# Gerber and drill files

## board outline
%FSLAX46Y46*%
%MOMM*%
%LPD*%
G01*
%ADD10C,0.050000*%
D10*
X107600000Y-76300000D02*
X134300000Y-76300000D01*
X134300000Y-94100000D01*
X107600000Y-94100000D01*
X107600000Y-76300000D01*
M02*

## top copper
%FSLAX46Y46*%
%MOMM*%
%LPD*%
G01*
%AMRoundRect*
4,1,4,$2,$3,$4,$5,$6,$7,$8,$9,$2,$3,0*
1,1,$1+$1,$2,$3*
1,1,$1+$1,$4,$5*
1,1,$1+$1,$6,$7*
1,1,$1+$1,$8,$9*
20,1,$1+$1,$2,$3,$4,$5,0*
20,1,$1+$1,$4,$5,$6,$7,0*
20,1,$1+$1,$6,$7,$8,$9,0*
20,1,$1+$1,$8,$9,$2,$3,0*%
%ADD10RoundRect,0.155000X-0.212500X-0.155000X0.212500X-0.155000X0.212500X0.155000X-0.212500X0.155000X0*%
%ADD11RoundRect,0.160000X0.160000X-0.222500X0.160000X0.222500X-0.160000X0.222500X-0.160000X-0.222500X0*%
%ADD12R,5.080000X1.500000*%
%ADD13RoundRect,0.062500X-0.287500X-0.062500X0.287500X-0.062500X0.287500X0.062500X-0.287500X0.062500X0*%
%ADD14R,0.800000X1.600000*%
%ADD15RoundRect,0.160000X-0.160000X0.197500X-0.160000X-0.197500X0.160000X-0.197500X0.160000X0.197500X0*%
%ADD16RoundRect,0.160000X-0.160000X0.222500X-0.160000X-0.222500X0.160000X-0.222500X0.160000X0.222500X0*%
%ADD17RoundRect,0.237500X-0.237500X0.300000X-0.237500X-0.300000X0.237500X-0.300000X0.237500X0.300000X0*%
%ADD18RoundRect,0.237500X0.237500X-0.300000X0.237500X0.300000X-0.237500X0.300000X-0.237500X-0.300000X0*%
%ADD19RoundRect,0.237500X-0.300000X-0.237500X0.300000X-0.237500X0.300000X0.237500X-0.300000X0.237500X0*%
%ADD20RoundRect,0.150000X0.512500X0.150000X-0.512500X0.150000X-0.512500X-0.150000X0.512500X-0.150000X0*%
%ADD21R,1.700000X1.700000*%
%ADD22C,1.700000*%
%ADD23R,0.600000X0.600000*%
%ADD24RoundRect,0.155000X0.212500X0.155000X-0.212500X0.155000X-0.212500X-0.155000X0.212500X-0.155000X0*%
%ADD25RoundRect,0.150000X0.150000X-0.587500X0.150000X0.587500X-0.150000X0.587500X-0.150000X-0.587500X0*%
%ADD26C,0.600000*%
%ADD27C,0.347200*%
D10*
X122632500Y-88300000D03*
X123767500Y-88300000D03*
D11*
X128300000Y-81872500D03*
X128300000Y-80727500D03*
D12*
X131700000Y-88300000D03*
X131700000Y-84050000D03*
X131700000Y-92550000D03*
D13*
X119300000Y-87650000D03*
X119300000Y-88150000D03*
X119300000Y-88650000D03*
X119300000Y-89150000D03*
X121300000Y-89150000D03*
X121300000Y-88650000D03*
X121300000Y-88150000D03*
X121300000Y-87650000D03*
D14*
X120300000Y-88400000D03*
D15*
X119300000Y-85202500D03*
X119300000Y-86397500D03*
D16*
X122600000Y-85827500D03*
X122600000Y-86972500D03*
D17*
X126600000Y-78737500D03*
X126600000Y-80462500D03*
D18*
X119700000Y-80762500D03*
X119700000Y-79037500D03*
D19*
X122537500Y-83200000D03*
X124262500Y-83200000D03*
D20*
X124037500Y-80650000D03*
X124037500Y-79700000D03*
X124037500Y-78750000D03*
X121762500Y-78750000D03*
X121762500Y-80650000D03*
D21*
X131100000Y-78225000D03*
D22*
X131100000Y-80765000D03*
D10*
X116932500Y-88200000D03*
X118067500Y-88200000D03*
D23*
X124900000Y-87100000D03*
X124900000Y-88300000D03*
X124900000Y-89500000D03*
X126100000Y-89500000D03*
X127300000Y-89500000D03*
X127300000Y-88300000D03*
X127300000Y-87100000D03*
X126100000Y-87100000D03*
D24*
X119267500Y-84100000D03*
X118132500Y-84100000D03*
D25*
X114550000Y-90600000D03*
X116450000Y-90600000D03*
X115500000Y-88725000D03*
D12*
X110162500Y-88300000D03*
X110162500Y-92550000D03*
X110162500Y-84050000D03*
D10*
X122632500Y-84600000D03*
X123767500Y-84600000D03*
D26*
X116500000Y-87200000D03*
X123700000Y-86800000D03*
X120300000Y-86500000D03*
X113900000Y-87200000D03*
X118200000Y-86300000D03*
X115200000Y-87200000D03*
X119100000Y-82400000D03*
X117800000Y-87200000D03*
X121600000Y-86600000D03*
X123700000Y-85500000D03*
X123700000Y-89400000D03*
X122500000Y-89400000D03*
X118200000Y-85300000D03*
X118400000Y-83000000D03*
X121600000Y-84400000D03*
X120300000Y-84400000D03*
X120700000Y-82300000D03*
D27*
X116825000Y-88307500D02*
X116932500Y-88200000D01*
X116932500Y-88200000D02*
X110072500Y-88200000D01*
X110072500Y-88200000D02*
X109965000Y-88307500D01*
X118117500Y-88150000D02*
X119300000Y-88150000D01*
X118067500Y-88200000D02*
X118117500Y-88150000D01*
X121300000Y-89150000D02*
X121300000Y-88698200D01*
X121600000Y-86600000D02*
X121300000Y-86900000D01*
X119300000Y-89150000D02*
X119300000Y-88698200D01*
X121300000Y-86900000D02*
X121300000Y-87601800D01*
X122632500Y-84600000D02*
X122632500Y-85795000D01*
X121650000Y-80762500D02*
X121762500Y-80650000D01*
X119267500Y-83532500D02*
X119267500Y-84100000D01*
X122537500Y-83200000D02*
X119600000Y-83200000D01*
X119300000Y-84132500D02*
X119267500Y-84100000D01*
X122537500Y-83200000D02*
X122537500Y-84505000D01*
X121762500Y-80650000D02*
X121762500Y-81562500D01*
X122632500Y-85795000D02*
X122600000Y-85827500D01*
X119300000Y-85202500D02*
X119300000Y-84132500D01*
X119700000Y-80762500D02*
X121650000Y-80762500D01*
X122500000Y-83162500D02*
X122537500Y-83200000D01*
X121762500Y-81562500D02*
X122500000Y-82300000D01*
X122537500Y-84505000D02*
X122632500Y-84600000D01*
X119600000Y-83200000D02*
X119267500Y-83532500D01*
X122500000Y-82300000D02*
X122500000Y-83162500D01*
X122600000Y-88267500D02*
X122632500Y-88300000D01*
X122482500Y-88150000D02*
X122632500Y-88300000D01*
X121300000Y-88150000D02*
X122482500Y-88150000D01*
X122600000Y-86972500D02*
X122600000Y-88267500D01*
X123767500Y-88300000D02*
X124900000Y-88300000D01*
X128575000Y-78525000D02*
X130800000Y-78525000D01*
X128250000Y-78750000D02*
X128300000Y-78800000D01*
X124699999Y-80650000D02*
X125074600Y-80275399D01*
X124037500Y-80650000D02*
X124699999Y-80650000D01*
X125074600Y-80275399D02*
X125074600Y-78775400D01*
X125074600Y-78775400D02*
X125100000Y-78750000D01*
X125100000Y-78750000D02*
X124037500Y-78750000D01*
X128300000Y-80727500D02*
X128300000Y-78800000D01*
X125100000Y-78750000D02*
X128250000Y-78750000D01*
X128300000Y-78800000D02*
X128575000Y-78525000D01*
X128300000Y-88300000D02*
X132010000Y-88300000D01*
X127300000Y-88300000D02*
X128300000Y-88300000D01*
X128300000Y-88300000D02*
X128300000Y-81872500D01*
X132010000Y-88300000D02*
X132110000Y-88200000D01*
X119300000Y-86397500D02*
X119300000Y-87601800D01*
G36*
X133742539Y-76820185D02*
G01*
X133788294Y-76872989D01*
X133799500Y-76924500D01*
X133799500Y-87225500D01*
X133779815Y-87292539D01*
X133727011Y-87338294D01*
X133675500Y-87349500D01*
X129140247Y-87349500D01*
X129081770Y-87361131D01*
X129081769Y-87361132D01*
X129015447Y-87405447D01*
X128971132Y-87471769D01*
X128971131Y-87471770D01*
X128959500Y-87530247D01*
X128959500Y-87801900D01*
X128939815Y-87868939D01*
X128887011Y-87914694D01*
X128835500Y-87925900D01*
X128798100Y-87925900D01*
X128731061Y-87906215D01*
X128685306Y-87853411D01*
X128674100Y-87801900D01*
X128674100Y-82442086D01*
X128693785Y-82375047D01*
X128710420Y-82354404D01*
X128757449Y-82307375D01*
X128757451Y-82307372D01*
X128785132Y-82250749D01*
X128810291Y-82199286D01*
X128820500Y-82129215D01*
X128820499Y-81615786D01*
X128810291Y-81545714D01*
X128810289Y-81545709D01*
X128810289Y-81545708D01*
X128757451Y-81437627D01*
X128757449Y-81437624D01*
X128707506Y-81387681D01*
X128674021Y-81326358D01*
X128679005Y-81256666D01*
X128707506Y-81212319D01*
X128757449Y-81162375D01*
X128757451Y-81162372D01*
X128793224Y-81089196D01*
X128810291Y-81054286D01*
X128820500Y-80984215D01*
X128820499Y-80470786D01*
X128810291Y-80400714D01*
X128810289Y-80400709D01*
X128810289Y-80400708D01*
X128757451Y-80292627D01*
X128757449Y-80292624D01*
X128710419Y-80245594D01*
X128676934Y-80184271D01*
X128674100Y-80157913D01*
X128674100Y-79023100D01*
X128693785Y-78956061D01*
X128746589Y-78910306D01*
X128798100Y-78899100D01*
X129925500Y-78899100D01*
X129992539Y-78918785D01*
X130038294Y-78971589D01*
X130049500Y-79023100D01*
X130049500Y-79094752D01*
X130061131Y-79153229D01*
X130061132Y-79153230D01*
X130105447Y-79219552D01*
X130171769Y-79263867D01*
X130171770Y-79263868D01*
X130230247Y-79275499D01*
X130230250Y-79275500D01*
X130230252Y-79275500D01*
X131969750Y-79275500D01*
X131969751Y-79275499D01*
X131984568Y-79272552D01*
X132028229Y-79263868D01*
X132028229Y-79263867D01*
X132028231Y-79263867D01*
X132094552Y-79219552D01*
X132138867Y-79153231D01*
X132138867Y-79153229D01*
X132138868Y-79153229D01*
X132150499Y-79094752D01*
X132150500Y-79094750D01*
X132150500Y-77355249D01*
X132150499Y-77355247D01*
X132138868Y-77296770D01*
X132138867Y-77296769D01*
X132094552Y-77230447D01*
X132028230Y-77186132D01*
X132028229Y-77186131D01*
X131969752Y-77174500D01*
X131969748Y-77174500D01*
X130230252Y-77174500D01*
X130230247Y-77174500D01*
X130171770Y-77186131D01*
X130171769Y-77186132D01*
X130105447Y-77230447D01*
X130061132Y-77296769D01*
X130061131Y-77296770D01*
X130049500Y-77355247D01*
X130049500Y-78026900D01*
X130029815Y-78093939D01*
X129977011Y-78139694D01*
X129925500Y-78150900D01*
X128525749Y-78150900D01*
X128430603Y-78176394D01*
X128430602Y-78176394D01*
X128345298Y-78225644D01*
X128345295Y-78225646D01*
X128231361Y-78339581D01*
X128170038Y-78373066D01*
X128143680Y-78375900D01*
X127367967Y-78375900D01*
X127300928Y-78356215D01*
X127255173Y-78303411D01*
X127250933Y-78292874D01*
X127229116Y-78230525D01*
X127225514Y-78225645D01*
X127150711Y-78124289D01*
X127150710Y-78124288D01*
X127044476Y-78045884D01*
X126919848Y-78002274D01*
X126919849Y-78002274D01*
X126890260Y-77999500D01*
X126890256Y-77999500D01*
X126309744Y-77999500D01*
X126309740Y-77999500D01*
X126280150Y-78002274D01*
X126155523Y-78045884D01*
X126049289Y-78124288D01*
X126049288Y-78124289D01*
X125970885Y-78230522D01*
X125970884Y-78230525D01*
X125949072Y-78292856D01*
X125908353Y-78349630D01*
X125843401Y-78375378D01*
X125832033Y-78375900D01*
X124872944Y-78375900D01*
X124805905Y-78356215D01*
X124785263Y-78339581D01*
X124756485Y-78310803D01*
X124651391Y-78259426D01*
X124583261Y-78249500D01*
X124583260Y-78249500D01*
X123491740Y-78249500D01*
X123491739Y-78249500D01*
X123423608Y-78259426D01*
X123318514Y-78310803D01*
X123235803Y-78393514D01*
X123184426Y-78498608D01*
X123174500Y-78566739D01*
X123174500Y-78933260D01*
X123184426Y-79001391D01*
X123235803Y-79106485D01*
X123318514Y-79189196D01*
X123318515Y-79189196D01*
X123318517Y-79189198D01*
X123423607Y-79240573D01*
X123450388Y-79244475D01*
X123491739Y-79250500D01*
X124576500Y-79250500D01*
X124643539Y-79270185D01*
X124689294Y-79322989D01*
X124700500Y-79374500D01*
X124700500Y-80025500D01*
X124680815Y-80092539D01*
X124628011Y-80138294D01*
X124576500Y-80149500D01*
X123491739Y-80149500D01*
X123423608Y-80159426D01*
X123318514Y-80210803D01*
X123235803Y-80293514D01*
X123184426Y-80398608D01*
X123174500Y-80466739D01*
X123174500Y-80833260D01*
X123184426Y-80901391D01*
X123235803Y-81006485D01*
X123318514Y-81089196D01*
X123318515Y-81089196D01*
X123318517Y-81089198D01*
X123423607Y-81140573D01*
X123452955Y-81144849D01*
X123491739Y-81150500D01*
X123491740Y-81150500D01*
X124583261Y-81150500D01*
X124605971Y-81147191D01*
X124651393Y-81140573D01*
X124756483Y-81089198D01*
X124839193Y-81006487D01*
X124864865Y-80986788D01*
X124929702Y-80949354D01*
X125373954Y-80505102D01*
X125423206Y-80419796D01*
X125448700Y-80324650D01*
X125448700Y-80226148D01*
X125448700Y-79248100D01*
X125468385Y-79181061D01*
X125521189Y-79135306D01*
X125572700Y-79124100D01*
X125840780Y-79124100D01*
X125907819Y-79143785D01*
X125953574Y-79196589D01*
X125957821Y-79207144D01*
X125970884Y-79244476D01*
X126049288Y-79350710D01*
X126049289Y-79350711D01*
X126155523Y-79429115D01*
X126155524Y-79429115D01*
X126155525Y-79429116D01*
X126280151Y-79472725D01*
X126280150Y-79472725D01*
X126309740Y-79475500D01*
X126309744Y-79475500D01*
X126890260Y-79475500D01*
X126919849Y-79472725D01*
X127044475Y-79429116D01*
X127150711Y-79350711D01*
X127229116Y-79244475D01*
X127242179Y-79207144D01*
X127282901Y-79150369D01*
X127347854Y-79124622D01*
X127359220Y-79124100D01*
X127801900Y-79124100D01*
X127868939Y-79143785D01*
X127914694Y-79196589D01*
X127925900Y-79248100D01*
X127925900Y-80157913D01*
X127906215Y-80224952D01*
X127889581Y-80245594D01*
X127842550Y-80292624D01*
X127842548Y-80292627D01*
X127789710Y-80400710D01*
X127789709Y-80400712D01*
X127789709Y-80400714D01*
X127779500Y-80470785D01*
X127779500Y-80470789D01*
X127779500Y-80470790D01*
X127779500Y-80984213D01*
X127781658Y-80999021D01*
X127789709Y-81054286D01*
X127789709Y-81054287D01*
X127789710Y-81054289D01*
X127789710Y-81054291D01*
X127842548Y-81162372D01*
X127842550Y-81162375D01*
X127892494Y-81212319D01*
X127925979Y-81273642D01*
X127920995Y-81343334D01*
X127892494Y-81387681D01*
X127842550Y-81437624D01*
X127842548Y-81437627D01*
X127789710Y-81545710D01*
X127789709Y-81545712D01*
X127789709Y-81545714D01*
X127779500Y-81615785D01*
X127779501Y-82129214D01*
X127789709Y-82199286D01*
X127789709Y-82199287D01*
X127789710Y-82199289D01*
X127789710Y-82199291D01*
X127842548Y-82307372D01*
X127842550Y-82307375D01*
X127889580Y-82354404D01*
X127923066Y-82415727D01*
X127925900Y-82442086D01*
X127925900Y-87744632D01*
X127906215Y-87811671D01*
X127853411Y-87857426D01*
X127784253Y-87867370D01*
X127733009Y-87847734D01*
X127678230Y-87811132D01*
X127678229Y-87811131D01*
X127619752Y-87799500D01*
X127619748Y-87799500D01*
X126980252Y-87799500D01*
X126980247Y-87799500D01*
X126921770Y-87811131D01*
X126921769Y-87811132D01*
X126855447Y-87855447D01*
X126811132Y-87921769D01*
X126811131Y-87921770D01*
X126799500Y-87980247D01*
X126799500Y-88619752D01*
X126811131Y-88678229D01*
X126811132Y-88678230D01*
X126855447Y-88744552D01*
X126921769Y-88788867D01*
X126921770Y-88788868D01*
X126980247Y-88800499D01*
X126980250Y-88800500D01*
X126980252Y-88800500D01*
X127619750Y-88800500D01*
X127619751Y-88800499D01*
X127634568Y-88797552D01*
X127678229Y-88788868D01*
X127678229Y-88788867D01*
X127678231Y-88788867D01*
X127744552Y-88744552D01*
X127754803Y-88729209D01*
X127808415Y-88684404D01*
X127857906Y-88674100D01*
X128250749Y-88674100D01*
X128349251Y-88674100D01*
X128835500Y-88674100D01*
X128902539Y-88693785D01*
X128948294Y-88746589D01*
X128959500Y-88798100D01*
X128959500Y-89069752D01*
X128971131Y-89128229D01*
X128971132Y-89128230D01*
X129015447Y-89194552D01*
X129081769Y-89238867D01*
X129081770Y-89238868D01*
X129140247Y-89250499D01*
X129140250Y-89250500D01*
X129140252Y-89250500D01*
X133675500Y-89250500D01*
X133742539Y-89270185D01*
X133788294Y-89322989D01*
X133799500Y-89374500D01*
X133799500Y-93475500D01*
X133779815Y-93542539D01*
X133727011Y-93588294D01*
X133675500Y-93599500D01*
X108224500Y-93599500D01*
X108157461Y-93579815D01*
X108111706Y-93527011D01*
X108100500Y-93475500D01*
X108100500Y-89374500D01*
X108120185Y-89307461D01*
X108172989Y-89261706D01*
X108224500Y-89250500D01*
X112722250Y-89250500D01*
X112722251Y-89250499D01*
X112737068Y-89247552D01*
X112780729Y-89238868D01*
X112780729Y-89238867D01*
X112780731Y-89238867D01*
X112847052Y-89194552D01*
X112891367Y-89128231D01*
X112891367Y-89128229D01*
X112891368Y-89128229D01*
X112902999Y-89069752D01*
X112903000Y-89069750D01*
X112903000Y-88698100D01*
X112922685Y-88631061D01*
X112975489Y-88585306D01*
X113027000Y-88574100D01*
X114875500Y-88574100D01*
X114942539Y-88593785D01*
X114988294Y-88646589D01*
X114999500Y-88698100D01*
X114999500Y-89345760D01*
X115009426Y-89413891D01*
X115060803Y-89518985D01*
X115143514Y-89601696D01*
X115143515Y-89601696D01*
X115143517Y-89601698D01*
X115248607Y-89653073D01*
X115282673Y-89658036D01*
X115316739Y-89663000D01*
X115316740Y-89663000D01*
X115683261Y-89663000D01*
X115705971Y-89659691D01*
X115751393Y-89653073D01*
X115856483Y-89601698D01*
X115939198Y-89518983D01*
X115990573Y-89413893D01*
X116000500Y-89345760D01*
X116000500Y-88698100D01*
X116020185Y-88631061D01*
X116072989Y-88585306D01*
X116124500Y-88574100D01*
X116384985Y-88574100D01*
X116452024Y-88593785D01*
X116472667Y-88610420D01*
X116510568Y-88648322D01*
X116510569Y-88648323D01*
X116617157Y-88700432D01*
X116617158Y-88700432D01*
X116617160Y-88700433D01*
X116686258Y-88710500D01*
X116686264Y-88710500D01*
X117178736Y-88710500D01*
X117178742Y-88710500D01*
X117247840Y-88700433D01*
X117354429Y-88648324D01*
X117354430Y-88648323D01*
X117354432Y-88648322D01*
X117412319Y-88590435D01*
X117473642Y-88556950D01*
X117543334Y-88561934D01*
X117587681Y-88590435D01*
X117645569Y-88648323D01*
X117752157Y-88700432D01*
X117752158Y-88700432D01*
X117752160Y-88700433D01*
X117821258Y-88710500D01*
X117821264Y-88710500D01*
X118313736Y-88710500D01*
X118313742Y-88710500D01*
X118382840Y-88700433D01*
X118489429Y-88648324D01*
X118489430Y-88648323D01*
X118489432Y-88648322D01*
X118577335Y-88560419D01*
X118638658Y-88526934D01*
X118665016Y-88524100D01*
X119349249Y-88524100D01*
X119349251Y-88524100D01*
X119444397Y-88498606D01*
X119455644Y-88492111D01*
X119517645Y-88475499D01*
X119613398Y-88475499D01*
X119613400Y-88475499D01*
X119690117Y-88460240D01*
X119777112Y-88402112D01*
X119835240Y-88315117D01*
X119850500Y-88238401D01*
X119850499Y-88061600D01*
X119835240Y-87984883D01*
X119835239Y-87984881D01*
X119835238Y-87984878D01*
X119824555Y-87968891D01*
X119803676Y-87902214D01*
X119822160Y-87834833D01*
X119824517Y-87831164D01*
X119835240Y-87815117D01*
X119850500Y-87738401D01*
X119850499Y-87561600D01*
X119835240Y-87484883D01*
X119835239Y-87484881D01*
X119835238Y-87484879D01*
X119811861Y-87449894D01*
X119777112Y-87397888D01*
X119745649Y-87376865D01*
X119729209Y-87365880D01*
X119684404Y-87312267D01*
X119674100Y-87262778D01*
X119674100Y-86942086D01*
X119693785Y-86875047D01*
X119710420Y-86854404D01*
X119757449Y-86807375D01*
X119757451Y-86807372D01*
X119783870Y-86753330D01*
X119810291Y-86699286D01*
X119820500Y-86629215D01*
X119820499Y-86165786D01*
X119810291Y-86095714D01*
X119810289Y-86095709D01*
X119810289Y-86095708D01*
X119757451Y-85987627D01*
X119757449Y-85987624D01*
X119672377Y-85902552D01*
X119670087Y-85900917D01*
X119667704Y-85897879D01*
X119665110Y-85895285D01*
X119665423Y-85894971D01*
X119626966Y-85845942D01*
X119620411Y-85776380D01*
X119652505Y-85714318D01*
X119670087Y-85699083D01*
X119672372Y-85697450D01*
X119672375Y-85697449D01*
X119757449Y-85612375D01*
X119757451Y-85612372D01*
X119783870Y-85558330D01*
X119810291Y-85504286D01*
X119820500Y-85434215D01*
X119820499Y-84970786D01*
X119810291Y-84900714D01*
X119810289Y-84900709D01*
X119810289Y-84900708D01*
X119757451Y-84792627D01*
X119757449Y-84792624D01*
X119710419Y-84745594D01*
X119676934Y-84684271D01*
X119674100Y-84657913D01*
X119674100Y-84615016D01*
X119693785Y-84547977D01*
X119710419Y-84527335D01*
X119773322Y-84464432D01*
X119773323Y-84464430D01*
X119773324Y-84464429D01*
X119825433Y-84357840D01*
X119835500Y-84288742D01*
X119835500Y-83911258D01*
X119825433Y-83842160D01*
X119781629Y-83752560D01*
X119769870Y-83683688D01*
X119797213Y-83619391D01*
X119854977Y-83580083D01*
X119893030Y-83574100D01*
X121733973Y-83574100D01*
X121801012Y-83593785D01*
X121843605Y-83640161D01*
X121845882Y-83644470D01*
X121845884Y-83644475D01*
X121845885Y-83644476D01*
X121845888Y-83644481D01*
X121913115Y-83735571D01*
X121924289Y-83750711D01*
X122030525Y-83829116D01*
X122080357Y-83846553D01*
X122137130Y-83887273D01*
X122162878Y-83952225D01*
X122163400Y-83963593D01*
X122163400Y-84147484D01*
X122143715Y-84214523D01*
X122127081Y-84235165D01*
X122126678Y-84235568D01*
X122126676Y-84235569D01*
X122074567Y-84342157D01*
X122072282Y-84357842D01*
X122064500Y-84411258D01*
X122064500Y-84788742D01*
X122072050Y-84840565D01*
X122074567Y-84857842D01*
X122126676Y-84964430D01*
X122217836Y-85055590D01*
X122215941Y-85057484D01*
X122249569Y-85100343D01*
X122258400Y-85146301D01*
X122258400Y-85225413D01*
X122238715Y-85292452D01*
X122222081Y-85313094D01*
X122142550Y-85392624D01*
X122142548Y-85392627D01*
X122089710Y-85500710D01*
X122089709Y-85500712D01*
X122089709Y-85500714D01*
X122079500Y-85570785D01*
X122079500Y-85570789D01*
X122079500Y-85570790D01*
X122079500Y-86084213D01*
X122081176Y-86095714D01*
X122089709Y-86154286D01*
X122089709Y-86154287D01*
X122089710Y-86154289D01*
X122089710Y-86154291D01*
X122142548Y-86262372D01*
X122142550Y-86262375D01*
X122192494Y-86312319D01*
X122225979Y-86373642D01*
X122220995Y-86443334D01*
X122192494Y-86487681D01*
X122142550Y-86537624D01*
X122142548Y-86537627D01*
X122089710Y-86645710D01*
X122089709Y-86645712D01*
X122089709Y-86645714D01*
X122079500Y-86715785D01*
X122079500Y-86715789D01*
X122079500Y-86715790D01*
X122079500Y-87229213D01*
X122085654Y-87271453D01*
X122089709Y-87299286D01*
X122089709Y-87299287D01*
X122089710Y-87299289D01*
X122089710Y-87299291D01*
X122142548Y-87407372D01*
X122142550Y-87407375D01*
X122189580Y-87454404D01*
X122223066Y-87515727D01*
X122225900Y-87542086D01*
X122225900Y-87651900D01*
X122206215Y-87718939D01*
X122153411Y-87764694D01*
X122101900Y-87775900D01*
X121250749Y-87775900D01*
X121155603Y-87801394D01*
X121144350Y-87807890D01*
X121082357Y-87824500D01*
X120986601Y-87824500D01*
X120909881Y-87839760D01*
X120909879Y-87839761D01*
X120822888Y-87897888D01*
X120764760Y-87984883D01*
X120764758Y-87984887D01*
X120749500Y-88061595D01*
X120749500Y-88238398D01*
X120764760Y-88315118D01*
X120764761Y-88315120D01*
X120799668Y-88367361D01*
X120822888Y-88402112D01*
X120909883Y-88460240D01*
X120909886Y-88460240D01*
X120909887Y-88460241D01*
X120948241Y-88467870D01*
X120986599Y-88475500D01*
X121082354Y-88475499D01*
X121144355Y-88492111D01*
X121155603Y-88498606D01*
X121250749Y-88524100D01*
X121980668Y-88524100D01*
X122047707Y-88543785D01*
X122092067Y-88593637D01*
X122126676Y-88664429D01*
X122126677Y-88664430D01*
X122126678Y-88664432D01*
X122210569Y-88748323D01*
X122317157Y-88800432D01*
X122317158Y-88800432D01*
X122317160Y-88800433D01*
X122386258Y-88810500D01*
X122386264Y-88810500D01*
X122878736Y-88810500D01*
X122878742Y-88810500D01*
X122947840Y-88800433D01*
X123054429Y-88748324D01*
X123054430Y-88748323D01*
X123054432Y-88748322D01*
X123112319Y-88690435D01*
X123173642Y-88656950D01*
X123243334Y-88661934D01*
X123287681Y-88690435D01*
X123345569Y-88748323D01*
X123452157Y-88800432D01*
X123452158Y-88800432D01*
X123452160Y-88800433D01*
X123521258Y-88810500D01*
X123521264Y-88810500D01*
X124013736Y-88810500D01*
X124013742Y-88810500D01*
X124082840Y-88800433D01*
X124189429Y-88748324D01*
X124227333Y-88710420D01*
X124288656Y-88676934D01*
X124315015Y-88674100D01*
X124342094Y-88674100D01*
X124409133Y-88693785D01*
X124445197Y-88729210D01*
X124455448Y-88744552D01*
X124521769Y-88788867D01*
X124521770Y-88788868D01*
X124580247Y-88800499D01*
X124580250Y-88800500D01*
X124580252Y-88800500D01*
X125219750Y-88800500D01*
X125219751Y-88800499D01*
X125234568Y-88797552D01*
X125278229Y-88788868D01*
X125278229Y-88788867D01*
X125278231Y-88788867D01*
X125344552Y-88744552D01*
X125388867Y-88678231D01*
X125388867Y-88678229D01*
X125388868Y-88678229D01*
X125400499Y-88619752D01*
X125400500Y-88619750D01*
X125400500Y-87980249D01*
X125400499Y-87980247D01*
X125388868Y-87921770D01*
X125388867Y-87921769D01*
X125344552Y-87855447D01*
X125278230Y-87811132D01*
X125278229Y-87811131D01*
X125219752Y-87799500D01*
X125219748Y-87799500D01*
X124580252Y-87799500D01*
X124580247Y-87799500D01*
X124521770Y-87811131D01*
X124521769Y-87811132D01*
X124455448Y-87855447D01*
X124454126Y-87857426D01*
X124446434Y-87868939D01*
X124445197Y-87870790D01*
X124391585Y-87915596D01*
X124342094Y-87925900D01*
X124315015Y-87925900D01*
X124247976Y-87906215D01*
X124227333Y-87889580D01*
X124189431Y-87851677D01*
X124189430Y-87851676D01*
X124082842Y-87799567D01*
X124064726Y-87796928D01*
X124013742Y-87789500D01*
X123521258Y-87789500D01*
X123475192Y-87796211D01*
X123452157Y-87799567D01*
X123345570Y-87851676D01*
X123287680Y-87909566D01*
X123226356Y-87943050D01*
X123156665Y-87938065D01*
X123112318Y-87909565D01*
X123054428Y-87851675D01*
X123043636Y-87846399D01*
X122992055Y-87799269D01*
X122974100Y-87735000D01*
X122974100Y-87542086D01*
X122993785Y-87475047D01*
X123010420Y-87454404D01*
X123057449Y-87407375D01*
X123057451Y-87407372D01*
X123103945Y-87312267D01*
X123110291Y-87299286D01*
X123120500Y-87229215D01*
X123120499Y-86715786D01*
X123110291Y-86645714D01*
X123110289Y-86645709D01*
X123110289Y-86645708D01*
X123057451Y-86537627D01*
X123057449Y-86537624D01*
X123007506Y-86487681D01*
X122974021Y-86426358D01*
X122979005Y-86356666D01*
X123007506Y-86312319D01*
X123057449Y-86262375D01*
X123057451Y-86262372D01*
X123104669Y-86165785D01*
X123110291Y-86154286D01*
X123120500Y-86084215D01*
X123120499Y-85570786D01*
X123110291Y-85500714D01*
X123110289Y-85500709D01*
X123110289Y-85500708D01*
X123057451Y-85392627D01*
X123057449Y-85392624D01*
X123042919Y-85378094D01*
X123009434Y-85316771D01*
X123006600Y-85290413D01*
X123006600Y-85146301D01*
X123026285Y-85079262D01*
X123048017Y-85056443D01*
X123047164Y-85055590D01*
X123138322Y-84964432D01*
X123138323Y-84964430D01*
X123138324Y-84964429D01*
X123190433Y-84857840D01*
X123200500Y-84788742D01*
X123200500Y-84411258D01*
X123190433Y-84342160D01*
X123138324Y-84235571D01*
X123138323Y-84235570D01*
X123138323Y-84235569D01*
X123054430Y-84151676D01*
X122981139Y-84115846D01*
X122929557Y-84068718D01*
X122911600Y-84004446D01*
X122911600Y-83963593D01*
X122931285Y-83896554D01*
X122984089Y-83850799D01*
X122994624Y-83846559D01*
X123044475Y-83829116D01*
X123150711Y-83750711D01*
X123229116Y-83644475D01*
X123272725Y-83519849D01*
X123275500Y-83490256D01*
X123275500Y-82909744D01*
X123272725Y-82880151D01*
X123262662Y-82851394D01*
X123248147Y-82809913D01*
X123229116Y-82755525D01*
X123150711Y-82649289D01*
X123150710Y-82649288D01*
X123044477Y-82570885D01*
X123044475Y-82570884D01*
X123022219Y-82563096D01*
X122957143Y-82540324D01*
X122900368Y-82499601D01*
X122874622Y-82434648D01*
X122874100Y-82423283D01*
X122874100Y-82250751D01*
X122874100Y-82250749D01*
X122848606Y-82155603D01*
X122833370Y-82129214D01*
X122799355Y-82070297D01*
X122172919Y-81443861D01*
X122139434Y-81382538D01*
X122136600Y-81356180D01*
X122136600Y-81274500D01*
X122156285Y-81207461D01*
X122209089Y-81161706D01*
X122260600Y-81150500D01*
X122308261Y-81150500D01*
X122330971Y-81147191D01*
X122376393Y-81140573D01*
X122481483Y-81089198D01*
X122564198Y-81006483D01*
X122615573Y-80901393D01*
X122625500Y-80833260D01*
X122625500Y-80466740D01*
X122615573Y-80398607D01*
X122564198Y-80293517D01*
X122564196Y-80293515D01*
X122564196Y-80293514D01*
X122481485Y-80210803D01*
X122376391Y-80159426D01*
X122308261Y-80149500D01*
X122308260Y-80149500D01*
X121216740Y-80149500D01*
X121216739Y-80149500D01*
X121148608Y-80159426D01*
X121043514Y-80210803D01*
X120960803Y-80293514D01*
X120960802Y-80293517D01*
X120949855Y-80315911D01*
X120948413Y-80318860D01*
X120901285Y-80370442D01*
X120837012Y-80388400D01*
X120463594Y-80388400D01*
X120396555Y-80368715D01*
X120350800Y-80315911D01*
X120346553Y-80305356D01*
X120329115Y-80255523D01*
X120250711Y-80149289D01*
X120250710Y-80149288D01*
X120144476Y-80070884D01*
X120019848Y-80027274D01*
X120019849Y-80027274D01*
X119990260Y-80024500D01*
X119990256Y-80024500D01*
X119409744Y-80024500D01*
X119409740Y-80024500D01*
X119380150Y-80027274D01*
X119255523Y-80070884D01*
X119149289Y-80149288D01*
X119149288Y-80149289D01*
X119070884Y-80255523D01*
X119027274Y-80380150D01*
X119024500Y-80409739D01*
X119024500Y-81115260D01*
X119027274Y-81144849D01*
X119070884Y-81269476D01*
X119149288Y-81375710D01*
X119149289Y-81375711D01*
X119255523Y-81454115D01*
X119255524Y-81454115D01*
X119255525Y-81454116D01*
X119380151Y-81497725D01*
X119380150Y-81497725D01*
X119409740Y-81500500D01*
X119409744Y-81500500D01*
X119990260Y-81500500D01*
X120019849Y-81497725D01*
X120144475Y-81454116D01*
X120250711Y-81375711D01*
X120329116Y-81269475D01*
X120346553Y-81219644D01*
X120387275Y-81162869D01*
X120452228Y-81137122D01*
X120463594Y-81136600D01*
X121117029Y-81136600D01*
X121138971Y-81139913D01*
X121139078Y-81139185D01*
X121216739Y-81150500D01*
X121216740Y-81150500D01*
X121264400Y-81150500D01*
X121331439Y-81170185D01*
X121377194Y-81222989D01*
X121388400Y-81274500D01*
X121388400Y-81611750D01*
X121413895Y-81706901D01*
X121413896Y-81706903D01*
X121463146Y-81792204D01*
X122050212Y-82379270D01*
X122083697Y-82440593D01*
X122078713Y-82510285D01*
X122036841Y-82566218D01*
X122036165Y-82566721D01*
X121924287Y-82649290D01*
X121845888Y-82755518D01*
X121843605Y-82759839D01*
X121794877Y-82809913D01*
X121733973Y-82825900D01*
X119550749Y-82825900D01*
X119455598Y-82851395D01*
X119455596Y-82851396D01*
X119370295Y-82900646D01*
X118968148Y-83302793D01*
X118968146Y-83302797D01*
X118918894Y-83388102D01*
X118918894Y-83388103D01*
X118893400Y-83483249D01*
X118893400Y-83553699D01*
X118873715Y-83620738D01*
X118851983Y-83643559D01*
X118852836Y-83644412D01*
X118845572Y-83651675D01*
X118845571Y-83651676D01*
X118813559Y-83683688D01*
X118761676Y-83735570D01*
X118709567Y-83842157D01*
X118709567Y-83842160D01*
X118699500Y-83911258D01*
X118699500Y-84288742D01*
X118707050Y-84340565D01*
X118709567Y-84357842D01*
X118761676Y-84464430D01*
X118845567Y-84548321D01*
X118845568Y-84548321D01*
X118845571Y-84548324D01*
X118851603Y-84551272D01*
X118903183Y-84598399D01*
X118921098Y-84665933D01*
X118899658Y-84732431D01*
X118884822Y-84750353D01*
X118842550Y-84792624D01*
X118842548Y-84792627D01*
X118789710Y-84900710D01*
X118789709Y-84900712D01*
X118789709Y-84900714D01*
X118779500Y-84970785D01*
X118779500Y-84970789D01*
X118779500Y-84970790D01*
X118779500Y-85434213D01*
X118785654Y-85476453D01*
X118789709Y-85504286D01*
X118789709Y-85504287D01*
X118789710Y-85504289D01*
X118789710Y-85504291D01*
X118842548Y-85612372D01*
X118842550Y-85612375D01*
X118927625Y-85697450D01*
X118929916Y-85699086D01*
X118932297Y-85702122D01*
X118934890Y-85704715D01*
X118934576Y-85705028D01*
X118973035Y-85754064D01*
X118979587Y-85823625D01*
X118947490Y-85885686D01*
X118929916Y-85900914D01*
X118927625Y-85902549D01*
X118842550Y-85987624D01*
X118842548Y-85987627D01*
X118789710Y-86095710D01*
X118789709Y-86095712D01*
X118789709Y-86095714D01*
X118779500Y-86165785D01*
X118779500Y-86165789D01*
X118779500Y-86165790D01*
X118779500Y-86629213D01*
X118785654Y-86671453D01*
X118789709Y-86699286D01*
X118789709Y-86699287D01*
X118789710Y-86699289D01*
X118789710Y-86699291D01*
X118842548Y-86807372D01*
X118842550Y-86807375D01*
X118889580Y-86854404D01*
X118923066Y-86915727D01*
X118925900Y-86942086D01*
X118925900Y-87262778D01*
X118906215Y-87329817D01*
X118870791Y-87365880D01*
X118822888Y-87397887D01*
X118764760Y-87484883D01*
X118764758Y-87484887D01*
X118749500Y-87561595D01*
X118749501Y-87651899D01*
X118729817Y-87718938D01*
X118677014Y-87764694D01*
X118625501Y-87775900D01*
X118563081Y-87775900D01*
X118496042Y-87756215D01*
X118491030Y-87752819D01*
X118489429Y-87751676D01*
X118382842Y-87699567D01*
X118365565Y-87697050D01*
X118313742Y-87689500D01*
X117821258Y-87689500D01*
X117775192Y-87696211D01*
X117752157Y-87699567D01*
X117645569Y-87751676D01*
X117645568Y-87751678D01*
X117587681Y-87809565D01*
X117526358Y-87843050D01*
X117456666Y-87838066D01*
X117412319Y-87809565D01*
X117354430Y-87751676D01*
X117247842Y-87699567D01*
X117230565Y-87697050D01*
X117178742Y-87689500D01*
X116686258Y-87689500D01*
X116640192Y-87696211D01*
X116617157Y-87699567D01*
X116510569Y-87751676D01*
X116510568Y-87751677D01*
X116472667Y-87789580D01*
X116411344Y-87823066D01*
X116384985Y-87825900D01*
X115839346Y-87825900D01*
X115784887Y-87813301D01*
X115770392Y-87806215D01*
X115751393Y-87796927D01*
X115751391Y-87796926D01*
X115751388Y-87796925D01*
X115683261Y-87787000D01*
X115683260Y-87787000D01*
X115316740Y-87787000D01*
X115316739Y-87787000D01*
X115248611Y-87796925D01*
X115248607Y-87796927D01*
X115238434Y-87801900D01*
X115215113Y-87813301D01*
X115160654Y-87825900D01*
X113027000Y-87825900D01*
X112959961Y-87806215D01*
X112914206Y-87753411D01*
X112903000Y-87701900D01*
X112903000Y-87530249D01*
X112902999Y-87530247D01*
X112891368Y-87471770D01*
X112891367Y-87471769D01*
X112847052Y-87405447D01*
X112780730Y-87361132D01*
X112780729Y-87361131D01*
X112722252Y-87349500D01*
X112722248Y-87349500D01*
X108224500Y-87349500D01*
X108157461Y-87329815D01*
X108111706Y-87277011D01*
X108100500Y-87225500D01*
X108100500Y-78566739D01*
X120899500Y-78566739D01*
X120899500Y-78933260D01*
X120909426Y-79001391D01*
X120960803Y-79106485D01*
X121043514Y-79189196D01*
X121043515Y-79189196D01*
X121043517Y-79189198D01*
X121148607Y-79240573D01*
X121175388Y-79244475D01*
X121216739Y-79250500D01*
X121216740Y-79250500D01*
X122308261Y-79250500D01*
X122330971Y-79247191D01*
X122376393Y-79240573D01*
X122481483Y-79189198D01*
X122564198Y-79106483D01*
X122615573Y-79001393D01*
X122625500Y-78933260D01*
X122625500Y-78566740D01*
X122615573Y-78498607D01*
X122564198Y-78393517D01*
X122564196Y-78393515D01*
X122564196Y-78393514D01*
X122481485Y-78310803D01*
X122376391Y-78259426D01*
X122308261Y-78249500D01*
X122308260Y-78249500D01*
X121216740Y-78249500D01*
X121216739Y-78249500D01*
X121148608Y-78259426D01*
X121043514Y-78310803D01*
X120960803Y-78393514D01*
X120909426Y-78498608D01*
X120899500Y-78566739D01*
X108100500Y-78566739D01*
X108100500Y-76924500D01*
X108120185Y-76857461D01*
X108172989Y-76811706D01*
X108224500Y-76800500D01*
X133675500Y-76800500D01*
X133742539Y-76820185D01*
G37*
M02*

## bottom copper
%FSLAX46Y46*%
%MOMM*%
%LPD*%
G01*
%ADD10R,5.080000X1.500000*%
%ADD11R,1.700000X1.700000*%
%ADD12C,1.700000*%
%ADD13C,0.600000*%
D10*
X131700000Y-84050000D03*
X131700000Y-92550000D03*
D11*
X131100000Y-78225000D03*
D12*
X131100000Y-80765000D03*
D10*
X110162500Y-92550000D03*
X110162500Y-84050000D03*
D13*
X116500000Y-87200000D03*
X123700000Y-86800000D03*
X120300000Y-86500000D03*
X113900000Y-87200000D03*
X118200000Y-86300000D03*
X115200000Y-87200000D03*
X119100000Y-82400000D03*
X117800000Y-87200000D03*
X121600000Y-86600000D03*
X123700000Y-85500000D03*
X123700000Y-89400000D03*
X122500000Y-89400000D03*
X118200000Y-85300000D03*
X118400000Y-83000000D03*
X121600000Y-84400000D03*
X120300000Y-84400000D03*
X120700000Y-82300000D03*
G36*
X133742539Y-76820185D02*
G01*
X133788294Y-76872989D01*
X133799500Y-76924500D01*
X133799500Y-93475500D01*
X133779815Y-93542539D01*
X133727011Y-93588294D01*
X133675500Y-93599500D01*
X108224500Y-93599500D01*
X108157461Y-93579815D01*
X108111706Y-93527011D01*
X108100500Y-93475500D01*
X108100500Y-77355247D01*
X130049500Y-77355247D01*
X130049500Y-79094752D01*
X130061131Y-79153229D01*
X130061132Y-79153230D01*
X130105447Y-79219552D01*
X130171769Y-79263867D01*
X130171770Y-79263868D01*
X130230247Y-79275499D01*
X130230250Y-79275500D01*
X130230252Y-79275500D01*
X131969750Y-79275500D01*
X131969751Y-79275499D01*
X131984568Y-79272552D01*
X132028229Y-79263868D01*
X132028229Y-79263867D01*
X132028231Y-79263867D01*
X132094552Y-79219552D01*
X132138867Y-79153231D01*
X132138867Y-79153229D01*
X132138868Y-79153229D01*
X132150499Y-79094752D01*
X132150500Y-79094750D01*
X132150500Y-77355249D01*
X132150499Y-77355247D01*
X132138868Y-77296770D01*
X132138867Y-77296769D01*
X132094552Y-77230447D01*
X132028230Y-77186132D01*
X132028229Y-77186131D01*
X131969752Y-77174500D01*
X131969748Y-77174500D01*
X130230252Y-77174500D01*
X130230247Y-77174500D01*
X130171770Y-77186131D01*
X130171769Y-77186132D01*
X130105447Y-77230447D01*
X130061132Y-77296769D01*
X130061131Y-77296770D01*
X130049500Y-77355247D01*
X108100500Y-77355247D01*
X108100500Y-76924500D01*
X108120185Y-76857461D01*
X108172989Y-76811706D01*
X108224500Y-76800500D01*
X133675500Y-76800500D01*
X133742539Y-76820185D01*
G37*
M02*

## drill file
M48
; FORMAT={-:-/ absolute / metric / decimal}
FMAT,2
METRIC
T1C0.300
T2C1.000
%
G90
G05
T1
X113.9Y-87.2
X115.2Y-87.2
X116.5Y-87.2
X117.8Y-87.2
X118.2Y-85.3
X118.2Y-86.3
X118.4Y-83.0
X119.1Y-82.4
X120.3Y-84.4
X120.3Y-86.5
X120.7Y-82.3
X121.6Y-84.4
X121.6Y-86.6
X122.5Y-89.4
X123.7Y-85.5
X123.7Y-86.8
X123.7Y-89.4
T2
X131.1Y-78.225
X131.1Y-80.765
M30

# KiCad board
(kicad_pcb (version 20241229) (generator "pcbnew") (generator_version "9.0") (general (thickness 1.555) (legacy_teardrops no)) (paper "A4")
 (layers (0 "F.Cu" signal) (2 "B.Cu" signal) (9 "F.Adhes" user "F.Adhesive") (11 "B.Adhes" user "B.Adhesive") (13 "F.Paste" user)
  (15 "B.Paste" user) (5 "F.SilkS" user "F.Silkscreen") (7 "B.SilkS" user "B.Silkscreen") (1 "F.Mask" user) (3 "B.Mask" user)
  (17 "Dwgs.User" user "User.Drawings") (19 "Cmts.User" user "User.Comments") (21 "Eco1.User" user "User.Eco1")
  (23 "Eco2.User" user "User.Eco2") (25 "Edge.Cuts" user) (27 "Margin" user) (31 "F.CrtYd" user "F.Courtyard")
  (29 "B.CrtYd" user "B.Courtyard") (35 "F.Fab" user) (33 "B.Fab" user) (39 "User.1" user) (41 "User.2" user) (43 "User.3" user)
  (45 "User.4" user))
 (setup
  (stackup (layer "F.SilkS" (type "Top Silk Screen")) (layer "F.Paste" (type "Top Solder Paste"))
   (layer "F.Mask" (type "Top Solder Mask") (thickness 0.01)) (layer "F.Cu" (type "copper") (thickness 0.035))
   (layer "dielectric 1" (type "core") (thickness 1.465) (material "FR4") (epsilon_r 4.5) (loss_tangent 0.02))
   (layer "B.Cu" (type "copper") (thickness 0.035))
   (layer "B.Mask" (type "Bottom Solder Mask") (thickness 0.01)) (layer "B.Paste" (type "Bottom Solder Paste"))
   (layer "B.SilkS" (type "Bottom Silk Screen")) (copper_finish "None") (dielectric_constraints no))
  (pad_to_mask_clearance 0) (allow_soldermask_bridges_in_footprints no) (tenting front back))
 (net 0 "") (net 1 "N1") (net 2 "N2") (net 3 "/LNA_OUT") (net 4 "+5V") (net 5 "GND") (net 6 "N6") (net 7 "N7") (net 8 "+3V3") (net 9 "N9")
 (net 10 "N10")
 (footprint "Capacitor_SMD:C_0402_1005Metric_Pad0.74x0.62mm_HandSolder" (layer "F.Cu") (at 123.2 88.3)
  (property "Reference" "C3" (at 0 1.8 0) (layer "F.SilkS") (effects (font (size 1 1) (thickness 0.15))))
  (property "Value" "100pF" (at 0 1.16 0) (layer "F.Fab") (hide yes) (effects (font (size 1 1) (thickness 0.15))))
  (pad "1" smd roundrect (at -0.5675 0) (size 0.735 0.62) (layers "F.Cu" "F.Mask" "F.Paste") (roundrect_rratio 0.25) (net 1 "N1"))
  (pad "2" smd roundrect (at 0.5675 0) (size 0.735 0.62) (layers "F.Cu" "F.Mask" "F.Paste") (roundrect_rratio 0.25) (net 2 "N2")))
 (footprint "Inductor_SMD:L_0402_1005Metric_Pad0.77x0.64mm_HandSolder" (layer "F.Cu") (at 128.3 81.3 90)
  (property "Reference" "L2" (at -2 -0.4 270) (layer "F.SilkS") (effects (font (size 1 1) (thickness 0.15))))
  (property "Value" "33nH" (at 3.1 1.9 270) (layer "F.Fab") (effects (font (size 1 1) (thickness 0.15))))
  (pad "1" smd roundrect (at -0.5725 0 90) (size 0.765 0.64) (layers "F.Cu" "F.Mask" "F.Paste") (roundrect_rratio 0.25) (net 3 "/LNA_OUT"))
  (pad "2" smd roundrect (at 0.5725 0 90) (size 0.765 0.64) (layers "F.Cu" "F.Mask" "F.Paste") (roundrect_rratio 0.25) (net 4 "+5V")))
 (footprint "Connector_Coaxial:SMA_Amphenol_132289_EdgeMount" (layer "F.Cu") (at 131.7 88.3)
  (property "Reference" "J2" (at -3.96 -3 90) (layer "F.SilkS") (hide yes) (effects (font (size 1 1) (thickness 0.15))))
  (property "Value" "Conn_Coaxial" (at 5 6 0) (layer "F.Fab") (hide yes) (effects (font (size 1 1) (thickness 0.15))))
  (pad "1" smd rect (at 0 0 90) (size 1.5 5.08) (layers "F.Cu" "F.Mask" "F.Paste") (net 3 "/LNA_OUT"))
  (pad "2" smd rect (at 0 -4.25 90) (size 1.5 5.08) (layers "F.Cu" "F.Mask" "F.Paste") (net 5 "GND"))
  (pad "2" smd rect (at 0 -4.25 90) (size 1.5 5.08) (layers "B.Cu" "B.Mask" "B.Paste") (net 5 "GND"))
  (pad "2" smd rect (at 0 4.25 90) (size 1.5 5.08) (layers "F.Cu" "F.Mask" "F.Paste") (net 5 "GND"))
  (pad "2" smd rect (at 0 4.25 90) (size 1.5 5.08) (layers "B.Cu" "B.Mask" "B.Paste") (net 5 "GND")))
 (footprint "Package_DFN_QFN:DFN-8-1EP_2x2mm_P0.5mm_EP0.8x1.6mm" (layer "F.Cu") (at 120.3 88.4)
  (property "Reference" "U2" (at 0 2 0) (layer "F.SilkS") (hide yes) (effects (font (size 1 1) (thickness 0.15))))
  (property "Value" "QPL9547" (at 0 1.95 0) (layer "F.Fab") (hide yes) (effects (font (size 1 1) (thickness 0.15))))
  (pad "" smd roundrect (at 0 0) (size 0.64 1.29) (layers "F.Paste") (roundrect_rratio 0.25))
  (pad "1" smd roundrect (at -1 -0.75) (size 0.7 0.25) (layers "F.Cu" "F.Mask" "F.Paste") (roundrect_rratio 0.25) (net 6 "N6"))
  (pad "2" smd roundrect (at -1 -0.25) (size 0.7 0.25) (layers "F.Cu" "F.Mask" "F.Paste") (roundrect_rratio 0.25) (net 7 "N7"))
  (pad "3" smd roundrect (at -1 0.25) (size 0.7 0.25) (layers "F.Cu" "F.Mask" "F.Paste") (roundrect_rratio 0.25) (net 5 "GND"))
  (pad "4" smd roundrect (at -1 0.75) (size 0.7 0.25) (layers "F.Cu" "F.Mask" "F.Paste") (roundrect_rratio 0.25) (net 5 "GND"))
  (pad "5" smd roundrect (at 1 0.75) (size 0.7 0.25) (layers "F.Cu" "F.Mask" "F.Paste") (roundrect_rratio 0.25) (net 5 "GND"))
  (pad "6" smd roundrect (at 1 0.25) (size 0.7 0.25) (layers "F.Cu" "F.Mask" "F.Paste") (roundrect_rratio 0.25) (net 5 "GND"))
  (pad "7" smd roundrect (at 1 -0.25) (size 0.7 0.25) (layers "F.Cu" "F.Mask" "F.Paste") (roundrect_rratio 0.25) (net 1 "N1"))
  (pad "8" smd roundrect (at 1 -0.75) (size 0.7 0.25) (layers "F.Cu" "F.Mask" "F.Paste") (roundrect_rratio 0.25) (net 5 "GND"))
  (pad "9" smd rect (at 0 0) (size 0.8 1.6) (layers "F.Cu" "F.Mask") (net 5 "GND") (zone_connect 2)))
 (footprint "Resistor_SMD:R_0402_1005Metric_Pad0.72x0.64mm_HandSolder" (layer "F.Cu") (at 119.3 85.8 -90)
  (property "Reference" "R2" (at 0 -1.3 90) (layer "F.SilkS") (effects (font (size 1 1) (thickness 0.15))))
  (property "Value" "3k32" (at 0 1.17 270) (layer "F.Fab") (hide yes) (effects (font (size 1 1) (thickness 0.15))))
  (pad "1" smd roundrect (at -0.5975 0 270) (size 0.715 0.64) (layers "F.Cu" "F.Mask" "F.Paste") (roundrect_rratio 0.25) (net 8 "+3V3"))
  (pad "2" smd roundrect (at 0.5975 0 270) (size 0.715 0.64) (layers "F.Cu" "F.Mask" "F.Paste") (roundrect_rratio 0.25) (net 6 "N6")))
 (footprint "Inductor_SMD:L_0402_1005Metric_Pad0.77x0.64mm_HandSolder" (layer "F.Cu") (at 122.6 86.4 -90)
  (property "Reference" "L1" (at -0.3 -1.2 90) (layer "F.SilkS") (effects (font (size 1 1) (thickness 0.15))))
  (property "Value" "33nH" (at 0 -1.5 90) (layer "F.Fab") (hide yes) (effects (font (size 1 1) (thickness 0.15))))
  (pad "1" smd roundrect (at -0.5725 0 270) (size 0.765 0.64) (layers "F.Cu" "F.Mask" "F.Paste") (roundrect_rratio 0.25) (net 8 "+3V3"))
  (pad "2" smd roundrect (at 0.5725 0 270) (size 0.765 0.64) (layers "F.Cu" "F.Mask" "F.Paste") (roundrect_rratio 0.25) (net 1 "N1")))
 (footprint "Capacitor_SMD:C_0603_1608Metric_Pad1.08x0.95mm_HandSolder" (layer "F.Cu") (at 126.6 79.6 -90)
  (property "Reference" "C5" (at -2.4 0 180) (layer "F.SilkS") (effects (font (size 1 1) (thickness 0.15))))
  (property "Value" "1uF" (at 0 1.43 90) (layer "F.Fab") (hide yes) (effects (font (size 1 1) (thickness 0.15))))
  (pad "1" smd roundrect (at -0.8625 0 270) (size 1.075 0.95) (layers "F.Cu" "F.Mask" "F.Paste") (roundrect_rratio 0.25) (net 4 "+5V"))
  (pad "2" smd roundrect (at 0.8625 0 270) (size 1.075 0.95) (layers "F.Cu" "F.Mask" "F.Paste") (roundrect_rratio 0.25) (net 5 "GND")))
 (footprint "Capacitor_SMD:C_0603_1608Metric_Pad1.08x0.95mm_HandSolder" (layer "F.Cu") (at 119.7 79.9 90)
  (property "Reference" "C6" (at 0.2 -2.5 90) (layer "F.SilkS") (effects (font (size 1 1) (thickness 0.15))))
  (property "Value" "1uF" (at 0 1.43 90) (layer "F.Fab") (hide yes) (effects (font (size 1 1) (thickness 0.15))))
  (pad "1" smd roundrect (at -0.8625 0 90) (size 1.075 0.95) (layers "F.Cu" "F.Mask" "F.Paste") (roundrect_rratio 0.25) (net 8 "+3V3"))
  (pad "2" smd roundrect (at 0.8625 0 90) (size 1.075 0.95) (layers "F.Cu" "F.Mask" "F.Paste") (roundrect_rratio 0.25) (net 5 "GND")))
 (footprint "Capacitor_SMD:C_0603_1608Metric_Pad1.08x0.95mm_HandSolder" (layer "F.Cu") (at 123.4 83.2)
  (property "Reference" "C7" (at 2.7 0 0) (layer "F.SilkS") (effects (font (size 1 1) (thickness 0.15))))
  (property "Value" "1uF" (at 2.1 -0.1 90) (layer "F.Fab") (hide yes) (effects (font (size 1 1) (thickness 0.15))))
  (pad "1" smd roundrect (at -0.8625 0) (size 1.075 0.95) (layers "F.Cu" "F.Mask" "F.Paste") (roundrect_rratio 0.25) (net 8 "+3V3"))
  (pad "2" smd roundrect (at 0.8625 0) (size 1.075 0.95) (layers "F.Cu" "F.Mask" "F.Paste") (roundrect_rratio 0.25) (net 5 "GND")))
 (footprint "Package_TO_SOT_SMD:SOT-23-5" (layer "F.Cu") (at 122.9 79.7 180)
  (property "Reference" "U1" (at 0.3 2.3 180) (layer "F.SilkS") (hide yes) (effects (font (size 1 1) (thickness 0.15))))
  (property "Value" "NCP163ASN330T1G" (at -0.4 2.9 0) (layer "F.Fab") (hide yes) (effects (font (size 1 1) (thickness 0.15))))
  (pad "1" smd roundrect (at -1.1375 -0.95 180) (size 1.325 0.6) (layers "F.Cu" "F.Mask" "F.Paste") (roundrect_rratio 0.25) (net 4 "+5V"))
  (pad "2" smd roundrect (at -1.1375 0 180) (size 1.325 0.6) (layers "F.Cu" "F.Mask" "F.Paste") (roundrect_rratio 0.25) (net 5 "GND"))
  (pad "3" smd roundrect (at -1.1375 0.95 180) (size 1.325 0.6) (layers "F.Cu" "F.Mask" "F.Paste") (roundrect_rratio 0.25) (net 4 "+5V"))
  (pad "4" smd roundrect (at 1.1375 0.95 180) (size 1.325 0.6) (layers "F.Cu" "F.Mask" "F.Paste") (roundrect_rratio 0.25) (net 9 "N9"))
  (pad "5" smd roundrect (at 1.1375 -0.95 180) (size 1.325 0.6) (layers "F.Cu" "F.Mask" "F.Paste") (roundrect_rratio 0.25) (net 8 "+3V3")))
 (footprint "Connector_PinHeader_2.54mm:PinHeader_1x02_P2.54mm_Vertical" (layer "F.Cu") (at 131.1 78.225)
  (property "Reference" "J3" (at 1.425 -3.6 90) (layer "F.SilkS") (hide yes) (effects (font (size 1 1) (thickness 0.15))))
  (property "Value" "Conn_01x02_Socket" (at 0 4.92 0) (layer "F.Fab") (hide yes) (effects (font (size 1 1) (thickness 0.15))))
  (pad "1" thru_hole rect (at 0 0) (size 1.7 1.7) (drill 1) (layers "*.Cu" "*.Mask") (remove_unused_layers no) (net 4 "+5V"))
  (pad "2" thru_hole circle (at 0 2.54) (size 1.7 1.7) (drill 1) (layers "*.Cu" "*.Mask") (remove_unused_layers no) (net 5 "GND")))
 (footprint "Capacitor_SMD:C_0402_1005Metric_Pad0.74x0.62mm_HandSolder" (layer "F.Cu") (at 117.5 88.2)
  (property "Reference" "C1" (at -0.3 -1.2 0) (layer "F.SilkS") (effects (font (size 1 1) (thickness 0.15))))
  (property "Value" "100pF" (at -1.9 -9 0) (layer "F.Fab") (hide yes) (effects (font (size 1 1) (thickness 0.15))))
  (pad "1" smd roundrect (at -0.5675 0) (size 0.735 0.62) (layers "F.Cu" "F.Mask" "F.Paste") (roundrect_rratio 0.25) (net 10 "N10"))
  (pad "2" smd roundrect (at 0.5675 0) (size 0.735 0.62) (layers "F.Cu" "F.Mask" "F.Paste") (roundrect_rratio 0.25) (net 7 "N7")))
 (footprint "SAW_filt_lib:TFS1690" (layer "F.Cu") (at 126.6 88.3 -90)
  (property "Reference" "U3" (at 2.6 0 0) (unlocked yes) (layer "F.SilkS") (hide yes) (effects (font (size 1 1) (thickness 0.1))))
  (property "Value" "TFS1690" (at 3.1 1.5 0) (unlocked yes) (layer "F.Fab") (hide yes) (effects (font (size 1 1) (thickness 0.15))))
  (pad "1" smd rect (at -1.2 1.7 270) (size 0.6 0.6) (layers "F.Cu" "F.Mask" "F.Paste") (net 5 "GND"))
  (pad "2" smd rect (at 0 1.7 270) (size 0.6 0.6) (layers "F.Cu" "F.Mask" "F.Paste") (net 2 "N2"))
  (pad "3" smd rect (at 1.2 1.7 270) (size 0.6 0.6) (layers "F.Cu" "F.Mask" "F.Paste") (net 5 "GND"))
  (pad "4" smd rect (at 1.2 0.5 270) (size 0.6 0.6) (layers "F.Cu" "F.Mask" "F.Paste") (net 5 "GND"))
  (pad "5" smd rect (at 1.2 -0.7 270) (size 0.6 0.6) (layers "F.Cu" "F.Mask" "F.Paste") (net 5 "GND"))
  (pad "6" smd rect (at 0 -0.7 270) (size 0.6 0.6) (layers "F.Cu" "F.Mask" "F.Paste") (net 3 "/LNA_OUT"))
  (pad "7" smd rect (at -1.2 -0.7 270) (size 0.6 0.6) (layers "F.Cu" "F.Mask" "F.Paste") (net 5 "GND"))
  (pad "8" smd rect (at -1.2 0.5 270) (size 0.6 0.6) (layers "F.Cu" "F.Mask" "F.Paste") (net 5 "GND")))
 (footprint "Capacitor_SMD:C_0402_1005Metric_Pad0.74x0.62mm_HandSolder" (layer "F.Cu") (at 118.7 84.1 180)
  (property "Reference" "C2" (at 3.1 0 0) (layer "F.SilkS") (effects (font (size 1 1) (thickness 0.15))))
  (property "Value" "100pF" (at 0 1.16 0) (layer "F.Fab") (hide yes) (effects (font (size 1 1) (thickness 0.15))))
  (pad "1" smd roundrect (at -0.5675 0 180) (size 0.735 0.62) (layers "F.Cu" "F.Mask" "F.Paste") (roundrect_rratio 0.25) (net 8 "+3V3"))
  (pad "2" smd roundrect (at 0.5675 0 180) (size 0.735 0.62) (layers "F.Cu" "F.Mask" "F.Paste") (roundrect_rratio 0.25) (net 5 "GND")))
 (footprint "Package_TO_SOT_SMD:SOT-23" (layer "F.Cu") (at 115.5 89.6625 90)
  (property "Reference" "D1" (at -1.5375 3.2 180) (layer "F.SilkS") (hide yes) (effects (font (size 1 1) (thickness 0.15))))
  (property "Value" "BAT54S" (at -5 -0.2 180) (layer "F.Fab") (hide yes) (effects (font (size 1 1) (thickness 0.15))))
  (pad "1" smd roundrect (at -0.9375 -0.95 90) (size 1.475 0.6) (layers "F.Cu" "F.Mask" "F.Paste") (roundrect_rratio 0.25) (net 5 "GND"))
  (pad "2" smd roundrect (at -0.9375 0.95 90) (size 1.475 0.6) (layers "F.Cu" "F.Mask" "F.Paste") (roundrect_rratio 0.25) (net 5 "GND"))
  (pad "3" smd roundrect (at 0.9375 0 90) (size 1.475 0.6) (layers "F.Cu" "F.Mask" "F.Paste") (roundrect_rratio 0.25) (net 10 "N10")))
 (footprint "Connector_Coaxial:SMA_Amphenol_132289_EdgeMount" (layer "F.Cu") (at 110.1625 88.3 180)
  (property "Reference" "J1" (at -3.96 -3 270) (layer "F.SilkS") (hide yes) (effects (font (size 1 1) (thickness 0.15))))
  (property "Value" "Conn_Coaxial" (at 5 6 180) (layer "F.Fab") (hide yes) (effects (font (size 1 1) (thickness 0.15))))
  (pad "1" smd rect (at 0 0 270) (size 1.5 5.08) (layers "F.Cu" "F.Mask" "F.Paste") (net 10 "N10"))
  (pad "2" smd rect (at 0 -4.25 270) (size 1.5 5.08) (layers "F.Cu" "F.Mask" "F.Paste") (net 5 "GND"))
  (pad "2" smd rect (at 0 -4.25 270) (size 1.5 5.08) (layers "B.Cu" "B.Mask" "B.Paste") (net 5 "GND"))
  (pad "2" smd rect (at 0 4.25 270) (size 1.5 5.08) (layers "F.Cu" "F.Mask" "F.Paste") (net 5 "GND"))
  (pad "2" smd rect (at 0 4.25 270) (size 1.5 5.08) (layers "B.Cu" "B.Mask" "B.Paste") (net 5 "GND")))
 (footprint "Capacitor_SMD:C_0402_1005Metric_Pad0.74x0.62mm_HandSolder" (layer "F.Cu") (at 123.2 84.6)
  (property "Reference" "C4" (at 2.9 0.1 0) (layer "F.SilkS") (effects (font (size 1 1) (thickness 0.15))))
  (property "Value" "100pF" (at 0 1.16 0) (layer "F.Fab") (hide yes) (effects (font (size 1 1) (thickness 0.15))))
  (pad "1" smd roundrect (at -0.5675 0) (size 0.735 0.62) (layers "F.Cu" "F.Mask" "F.Paste") (roundrect_rratio 0.25) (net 8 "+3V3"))
  (pad "2" smd roundrect (at 0.5675 0) (size 0.735 0.62) (layers "F.Cu" "F.Mask" "F.Paste") (roundrect_rratio 0.25) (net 5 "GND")))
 (gr_rect (start 107.6 76.3) (end 134.3 94.1) (stroke (width 0.05) (type default)) (fill no) (layer "Edge.Cuts"))
 (segment (start 116.825 88.3075) (end 116.9325 88.2) (width 0.3472) (layer "F.Cu") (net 10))
 (segment (start 116.9325 88.2) (end 110.0725 88.2) (width 0.3472) (layer "F.Cu") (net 10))
 (segment (start 110.0725 88.2) (end 109.965 88.3075) (width 0.3472) (layer "F.Cu") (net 10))
 (segment (start 118.1175 88.15) (end 119.3 88.15) (width 0.3472) (layer "F.Cu") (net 7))
 (segment (start 118.0675 88.2) (end 118.1175 88.15) (width 0.3472) (layer "F.Cu") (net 7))
 (segment (start 121.3 89.15) (end 121.3 88.6982) (width 0.3472) (layer "F.Cu") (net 5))
 (segment (start 121.6 86.6) (end 121.3 86.9) (width 0.3472) (layer "F.Cu") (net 5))
 (segment (start 119.3 89.15) (end 119.3 88.6982) (width 0.3472) (layer "F.Cu") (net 5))
 (segment (start 121.3 86.9) (end 121.3 87.6018) (width 0.3472) (layer "F.Cu") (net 5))
 (via (at 116.5 87.2) (size 0.6) (drill 0.3) (layers "F.Cu" "B.Cu") (free yes) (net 5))
 (via (at 123.7 86.8) (size 0.6) (drill 0.3) (layers "F.Cu" "B.Cu") (free yes) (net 5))
 (via (at 120.3 86.5) (size 0.6) (drill 0.3) (layers "F.Cu" "B.Cu") (free yes) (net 5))
 (via (at 113.9 87.2) (size 0.6) (drill 0.3) (layers "F.Cu" "B.Cu") (free yes) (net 5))
 (via (at 118.2 86.3) (size 0.6) (drill 0.3) (layers "F.Cu" "B.Cu") (free yes) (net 5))
 (via (at 115.2 87.2) (size 0.6) (drill 0.3) (layers "F.Cu" "B.Cu") (free yes) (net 5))
 (via (at 119.1 82.4) (size 0.6) (drill 0.3) (layers "F.Cu" "B.Cu") (free yes) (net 5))
 (via (at 117.8 87.2) (size 0.6) (drill 0.3) (layers "F.Cu" "B.Cu") (free yes) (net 5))
 (via (at 121.6 86.6) (size 0.6) (drill 0.3) (layers "F.Cu" "B.Cu") (free yes) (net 5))
 (via (at 123.7 85.5) (size 0.6) (drill 0.3) (layers "F.Cu" "B.Cu") (free yes) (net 5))
 (via (at 123.7 89.4) (size 0.6) (drill 0.3) (layers "F.Cu" "B.Cu") (free yes) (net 5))
 (via (at 122.5 89.4) (size 0.6) (drill 0.3) (layers "F.Cu" "B.Cu") (free yes) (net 5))
 (via (at 118.2 85.3) (size 0.6) (drill 0.3) (layers "F.Cu" "B.Cu") (free yes) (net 5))
 (via (at 118.4 83) (size 0.6) (drill 0.3) (layers "F.Cu" "B.Cu") (free yes) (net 5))
 (via (at 121.6 84.4) (size 0.6) (drill 0.3) (layers "F.Cu" "B.Cu") (free yes) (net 5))
 (via (at 120.3 84.4) (size 0.6) (drill 0.3) (layers "F.Cu" "B.Cu") (free yes) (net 5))
 (via (at 120.7 82.3) (size 0.6) (drill 0.3) (layers "F.Cu" "B.Cu") (free yes) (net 5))
 (segment (start 122.6325 84.6) (end 122.6325 85.795) (width 0.3472) (layer "F.Cu") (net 8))
 (segment (start 121.65 80.7625) (end 121.7625 80.65) (width 0.3472) (layer "F.Cu") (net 8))
 (segment (start 119.2675 83.5325) (end 119.2675 84.1) (width 0.3472) (layer "F.Cu") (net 8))
 (segment (start 122.5375 83.2) (end 119.6 83.2) (width 0.3472) (layer "F.Cu") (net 8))
 (segment (start 119.3 84.1325) (end 119.2675 84.1) (width 0.3472) (layer "F.Cu") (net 8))
 (segment (start 122.5375 83.2) (end 122.5375 84.505) (width 0.3472) (layer "F.Cu") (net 8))
 (segment (start 121.7625 80.65) (end 121.7625 81.5625) (width 0.3472) (layer "F.Cu") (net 8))
 (segment (start 122.6325 85.795) (end 122.6 85.8275) (width 0.3472) (layer "F.Cu") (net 8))
 (segment (start 119.3 85.2025) (end 119.3 84.1325) (width 0.3472) (layer "F.Cu") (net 8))
 (segment (start 119.7 80.7625) (end 121.65 80.7625) (width 0.3472) (layer "F.Cu") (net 8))
 (segment (start 122.5 83.1625) (end 122.5375 83.2) (width 0.3472) (layer "F.Cu") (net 8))
 (segment (start 121.7625 81.5625) (end 122.5 82.3) (width 0.3472) (layer "F.Cu") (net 8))
 (segment (start 122.5375 84.505) (end 122.6325 84.6) (width 0.3472) (layer "F.Cu") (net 8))
 (segment (start 119.6 83.2) (end 119.2675 83.5325) (width 0.3472) (layer "F.Cu") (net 8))
 (segment (start 122.5 82.3) (end 122.5 83.1625) (width 0.3472) (layer "F.Cu") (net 8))
 (segment (start 122.6 88.2675) (end 122.6325 88.3) (width 0.3472) (layer "F.Cu") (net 1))
 (segment (start 122.4825 88.15) (end 122.6325 88.3) (width 0.3472) (layer "F.Cu") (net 1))
 (segment (start 121.3 88.15) (end 122.4825 88.15) (width 0.3472) (layer "F.Cu") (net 1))
 (segment (start 122.6 86.9725) (end 122.6 88.2675) (width 0.3472) (layer "F.Cu") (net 1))
 (segment (start 123.7675 88.3) (end 124.9 88.3) (width 0.3472) (layer "F.Cu") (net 2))
 (segment (start 128.575 78.525) (end 130.8 78.525) (width 0.3472) (layer "F.Cu") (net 4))
 (segment (start 128.25 78.75) (end 128.3 78.8) (width 0.3472) (layer "F.Cu") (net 4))
 (segment (start 124.699999 80.65) (end 125.0746 80.275399) (width 0.3472) (layer "F.Cu") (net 4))
 (segment (start 124.0375 80.65) (end 124.699999 80.65) (width 0.3472) (layer "F.Cu") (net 4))
 (segment (start 125.0746 80.275399) (end 125.0746 78.7754) (width 0.3472) (layer "F.Cu") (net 4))
 (segment (start 125.0746 78.7754) (end 125.1 78.75) (width 0.3472) (layer "F.Cu") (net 4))
 (segment (start 125.1 78.75) (end 124.0375 78.75) (width 0.3472) (layer "F.Cu") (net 4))
 (segment (start 128.3 80.7275) (end 128.3 78.8) (width 0.3472) (layer "F.Cu") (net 4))
 (segment (start 125.1 78.75) (end 128.25 78.75) (width 0.3472) (layer "F.Cu") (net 4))
 (segment (start 128.3 78.8) (end 128.575 78.525) (width 0.3472) (layer "F.Cu") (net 4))
 (segment (start 128.3 88.3) (end 132.01 88.3) (width 0.3472) (layer "F.Cu") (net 3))
 (segment (start 127.3 88.3) (end 128.3 88.3) (width 0.3472) (layer "F.Cu") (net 3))
 (segment (start 128.3 88.3) (end 128.3 81.8725) (width 0.3472) (layer "F.Cu") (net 3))
 (segment (start 132.01 88.3) (end 132.11 88.2) (width 0.3472) (layer "F.Cu") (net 3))
 (segment (start 119.3 86.3975) (end 119.3 87.6018) (width 0.3472) (layer "F.Cu") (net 6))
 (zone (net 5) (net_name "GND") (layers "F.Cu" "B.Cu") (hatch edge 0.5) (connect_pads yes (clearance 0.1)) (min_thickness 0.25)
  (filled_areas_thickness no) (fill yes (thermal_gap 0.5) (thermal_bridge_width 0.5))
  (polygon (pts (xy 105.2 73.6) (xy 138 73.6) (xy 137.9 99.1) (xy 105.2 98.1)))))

